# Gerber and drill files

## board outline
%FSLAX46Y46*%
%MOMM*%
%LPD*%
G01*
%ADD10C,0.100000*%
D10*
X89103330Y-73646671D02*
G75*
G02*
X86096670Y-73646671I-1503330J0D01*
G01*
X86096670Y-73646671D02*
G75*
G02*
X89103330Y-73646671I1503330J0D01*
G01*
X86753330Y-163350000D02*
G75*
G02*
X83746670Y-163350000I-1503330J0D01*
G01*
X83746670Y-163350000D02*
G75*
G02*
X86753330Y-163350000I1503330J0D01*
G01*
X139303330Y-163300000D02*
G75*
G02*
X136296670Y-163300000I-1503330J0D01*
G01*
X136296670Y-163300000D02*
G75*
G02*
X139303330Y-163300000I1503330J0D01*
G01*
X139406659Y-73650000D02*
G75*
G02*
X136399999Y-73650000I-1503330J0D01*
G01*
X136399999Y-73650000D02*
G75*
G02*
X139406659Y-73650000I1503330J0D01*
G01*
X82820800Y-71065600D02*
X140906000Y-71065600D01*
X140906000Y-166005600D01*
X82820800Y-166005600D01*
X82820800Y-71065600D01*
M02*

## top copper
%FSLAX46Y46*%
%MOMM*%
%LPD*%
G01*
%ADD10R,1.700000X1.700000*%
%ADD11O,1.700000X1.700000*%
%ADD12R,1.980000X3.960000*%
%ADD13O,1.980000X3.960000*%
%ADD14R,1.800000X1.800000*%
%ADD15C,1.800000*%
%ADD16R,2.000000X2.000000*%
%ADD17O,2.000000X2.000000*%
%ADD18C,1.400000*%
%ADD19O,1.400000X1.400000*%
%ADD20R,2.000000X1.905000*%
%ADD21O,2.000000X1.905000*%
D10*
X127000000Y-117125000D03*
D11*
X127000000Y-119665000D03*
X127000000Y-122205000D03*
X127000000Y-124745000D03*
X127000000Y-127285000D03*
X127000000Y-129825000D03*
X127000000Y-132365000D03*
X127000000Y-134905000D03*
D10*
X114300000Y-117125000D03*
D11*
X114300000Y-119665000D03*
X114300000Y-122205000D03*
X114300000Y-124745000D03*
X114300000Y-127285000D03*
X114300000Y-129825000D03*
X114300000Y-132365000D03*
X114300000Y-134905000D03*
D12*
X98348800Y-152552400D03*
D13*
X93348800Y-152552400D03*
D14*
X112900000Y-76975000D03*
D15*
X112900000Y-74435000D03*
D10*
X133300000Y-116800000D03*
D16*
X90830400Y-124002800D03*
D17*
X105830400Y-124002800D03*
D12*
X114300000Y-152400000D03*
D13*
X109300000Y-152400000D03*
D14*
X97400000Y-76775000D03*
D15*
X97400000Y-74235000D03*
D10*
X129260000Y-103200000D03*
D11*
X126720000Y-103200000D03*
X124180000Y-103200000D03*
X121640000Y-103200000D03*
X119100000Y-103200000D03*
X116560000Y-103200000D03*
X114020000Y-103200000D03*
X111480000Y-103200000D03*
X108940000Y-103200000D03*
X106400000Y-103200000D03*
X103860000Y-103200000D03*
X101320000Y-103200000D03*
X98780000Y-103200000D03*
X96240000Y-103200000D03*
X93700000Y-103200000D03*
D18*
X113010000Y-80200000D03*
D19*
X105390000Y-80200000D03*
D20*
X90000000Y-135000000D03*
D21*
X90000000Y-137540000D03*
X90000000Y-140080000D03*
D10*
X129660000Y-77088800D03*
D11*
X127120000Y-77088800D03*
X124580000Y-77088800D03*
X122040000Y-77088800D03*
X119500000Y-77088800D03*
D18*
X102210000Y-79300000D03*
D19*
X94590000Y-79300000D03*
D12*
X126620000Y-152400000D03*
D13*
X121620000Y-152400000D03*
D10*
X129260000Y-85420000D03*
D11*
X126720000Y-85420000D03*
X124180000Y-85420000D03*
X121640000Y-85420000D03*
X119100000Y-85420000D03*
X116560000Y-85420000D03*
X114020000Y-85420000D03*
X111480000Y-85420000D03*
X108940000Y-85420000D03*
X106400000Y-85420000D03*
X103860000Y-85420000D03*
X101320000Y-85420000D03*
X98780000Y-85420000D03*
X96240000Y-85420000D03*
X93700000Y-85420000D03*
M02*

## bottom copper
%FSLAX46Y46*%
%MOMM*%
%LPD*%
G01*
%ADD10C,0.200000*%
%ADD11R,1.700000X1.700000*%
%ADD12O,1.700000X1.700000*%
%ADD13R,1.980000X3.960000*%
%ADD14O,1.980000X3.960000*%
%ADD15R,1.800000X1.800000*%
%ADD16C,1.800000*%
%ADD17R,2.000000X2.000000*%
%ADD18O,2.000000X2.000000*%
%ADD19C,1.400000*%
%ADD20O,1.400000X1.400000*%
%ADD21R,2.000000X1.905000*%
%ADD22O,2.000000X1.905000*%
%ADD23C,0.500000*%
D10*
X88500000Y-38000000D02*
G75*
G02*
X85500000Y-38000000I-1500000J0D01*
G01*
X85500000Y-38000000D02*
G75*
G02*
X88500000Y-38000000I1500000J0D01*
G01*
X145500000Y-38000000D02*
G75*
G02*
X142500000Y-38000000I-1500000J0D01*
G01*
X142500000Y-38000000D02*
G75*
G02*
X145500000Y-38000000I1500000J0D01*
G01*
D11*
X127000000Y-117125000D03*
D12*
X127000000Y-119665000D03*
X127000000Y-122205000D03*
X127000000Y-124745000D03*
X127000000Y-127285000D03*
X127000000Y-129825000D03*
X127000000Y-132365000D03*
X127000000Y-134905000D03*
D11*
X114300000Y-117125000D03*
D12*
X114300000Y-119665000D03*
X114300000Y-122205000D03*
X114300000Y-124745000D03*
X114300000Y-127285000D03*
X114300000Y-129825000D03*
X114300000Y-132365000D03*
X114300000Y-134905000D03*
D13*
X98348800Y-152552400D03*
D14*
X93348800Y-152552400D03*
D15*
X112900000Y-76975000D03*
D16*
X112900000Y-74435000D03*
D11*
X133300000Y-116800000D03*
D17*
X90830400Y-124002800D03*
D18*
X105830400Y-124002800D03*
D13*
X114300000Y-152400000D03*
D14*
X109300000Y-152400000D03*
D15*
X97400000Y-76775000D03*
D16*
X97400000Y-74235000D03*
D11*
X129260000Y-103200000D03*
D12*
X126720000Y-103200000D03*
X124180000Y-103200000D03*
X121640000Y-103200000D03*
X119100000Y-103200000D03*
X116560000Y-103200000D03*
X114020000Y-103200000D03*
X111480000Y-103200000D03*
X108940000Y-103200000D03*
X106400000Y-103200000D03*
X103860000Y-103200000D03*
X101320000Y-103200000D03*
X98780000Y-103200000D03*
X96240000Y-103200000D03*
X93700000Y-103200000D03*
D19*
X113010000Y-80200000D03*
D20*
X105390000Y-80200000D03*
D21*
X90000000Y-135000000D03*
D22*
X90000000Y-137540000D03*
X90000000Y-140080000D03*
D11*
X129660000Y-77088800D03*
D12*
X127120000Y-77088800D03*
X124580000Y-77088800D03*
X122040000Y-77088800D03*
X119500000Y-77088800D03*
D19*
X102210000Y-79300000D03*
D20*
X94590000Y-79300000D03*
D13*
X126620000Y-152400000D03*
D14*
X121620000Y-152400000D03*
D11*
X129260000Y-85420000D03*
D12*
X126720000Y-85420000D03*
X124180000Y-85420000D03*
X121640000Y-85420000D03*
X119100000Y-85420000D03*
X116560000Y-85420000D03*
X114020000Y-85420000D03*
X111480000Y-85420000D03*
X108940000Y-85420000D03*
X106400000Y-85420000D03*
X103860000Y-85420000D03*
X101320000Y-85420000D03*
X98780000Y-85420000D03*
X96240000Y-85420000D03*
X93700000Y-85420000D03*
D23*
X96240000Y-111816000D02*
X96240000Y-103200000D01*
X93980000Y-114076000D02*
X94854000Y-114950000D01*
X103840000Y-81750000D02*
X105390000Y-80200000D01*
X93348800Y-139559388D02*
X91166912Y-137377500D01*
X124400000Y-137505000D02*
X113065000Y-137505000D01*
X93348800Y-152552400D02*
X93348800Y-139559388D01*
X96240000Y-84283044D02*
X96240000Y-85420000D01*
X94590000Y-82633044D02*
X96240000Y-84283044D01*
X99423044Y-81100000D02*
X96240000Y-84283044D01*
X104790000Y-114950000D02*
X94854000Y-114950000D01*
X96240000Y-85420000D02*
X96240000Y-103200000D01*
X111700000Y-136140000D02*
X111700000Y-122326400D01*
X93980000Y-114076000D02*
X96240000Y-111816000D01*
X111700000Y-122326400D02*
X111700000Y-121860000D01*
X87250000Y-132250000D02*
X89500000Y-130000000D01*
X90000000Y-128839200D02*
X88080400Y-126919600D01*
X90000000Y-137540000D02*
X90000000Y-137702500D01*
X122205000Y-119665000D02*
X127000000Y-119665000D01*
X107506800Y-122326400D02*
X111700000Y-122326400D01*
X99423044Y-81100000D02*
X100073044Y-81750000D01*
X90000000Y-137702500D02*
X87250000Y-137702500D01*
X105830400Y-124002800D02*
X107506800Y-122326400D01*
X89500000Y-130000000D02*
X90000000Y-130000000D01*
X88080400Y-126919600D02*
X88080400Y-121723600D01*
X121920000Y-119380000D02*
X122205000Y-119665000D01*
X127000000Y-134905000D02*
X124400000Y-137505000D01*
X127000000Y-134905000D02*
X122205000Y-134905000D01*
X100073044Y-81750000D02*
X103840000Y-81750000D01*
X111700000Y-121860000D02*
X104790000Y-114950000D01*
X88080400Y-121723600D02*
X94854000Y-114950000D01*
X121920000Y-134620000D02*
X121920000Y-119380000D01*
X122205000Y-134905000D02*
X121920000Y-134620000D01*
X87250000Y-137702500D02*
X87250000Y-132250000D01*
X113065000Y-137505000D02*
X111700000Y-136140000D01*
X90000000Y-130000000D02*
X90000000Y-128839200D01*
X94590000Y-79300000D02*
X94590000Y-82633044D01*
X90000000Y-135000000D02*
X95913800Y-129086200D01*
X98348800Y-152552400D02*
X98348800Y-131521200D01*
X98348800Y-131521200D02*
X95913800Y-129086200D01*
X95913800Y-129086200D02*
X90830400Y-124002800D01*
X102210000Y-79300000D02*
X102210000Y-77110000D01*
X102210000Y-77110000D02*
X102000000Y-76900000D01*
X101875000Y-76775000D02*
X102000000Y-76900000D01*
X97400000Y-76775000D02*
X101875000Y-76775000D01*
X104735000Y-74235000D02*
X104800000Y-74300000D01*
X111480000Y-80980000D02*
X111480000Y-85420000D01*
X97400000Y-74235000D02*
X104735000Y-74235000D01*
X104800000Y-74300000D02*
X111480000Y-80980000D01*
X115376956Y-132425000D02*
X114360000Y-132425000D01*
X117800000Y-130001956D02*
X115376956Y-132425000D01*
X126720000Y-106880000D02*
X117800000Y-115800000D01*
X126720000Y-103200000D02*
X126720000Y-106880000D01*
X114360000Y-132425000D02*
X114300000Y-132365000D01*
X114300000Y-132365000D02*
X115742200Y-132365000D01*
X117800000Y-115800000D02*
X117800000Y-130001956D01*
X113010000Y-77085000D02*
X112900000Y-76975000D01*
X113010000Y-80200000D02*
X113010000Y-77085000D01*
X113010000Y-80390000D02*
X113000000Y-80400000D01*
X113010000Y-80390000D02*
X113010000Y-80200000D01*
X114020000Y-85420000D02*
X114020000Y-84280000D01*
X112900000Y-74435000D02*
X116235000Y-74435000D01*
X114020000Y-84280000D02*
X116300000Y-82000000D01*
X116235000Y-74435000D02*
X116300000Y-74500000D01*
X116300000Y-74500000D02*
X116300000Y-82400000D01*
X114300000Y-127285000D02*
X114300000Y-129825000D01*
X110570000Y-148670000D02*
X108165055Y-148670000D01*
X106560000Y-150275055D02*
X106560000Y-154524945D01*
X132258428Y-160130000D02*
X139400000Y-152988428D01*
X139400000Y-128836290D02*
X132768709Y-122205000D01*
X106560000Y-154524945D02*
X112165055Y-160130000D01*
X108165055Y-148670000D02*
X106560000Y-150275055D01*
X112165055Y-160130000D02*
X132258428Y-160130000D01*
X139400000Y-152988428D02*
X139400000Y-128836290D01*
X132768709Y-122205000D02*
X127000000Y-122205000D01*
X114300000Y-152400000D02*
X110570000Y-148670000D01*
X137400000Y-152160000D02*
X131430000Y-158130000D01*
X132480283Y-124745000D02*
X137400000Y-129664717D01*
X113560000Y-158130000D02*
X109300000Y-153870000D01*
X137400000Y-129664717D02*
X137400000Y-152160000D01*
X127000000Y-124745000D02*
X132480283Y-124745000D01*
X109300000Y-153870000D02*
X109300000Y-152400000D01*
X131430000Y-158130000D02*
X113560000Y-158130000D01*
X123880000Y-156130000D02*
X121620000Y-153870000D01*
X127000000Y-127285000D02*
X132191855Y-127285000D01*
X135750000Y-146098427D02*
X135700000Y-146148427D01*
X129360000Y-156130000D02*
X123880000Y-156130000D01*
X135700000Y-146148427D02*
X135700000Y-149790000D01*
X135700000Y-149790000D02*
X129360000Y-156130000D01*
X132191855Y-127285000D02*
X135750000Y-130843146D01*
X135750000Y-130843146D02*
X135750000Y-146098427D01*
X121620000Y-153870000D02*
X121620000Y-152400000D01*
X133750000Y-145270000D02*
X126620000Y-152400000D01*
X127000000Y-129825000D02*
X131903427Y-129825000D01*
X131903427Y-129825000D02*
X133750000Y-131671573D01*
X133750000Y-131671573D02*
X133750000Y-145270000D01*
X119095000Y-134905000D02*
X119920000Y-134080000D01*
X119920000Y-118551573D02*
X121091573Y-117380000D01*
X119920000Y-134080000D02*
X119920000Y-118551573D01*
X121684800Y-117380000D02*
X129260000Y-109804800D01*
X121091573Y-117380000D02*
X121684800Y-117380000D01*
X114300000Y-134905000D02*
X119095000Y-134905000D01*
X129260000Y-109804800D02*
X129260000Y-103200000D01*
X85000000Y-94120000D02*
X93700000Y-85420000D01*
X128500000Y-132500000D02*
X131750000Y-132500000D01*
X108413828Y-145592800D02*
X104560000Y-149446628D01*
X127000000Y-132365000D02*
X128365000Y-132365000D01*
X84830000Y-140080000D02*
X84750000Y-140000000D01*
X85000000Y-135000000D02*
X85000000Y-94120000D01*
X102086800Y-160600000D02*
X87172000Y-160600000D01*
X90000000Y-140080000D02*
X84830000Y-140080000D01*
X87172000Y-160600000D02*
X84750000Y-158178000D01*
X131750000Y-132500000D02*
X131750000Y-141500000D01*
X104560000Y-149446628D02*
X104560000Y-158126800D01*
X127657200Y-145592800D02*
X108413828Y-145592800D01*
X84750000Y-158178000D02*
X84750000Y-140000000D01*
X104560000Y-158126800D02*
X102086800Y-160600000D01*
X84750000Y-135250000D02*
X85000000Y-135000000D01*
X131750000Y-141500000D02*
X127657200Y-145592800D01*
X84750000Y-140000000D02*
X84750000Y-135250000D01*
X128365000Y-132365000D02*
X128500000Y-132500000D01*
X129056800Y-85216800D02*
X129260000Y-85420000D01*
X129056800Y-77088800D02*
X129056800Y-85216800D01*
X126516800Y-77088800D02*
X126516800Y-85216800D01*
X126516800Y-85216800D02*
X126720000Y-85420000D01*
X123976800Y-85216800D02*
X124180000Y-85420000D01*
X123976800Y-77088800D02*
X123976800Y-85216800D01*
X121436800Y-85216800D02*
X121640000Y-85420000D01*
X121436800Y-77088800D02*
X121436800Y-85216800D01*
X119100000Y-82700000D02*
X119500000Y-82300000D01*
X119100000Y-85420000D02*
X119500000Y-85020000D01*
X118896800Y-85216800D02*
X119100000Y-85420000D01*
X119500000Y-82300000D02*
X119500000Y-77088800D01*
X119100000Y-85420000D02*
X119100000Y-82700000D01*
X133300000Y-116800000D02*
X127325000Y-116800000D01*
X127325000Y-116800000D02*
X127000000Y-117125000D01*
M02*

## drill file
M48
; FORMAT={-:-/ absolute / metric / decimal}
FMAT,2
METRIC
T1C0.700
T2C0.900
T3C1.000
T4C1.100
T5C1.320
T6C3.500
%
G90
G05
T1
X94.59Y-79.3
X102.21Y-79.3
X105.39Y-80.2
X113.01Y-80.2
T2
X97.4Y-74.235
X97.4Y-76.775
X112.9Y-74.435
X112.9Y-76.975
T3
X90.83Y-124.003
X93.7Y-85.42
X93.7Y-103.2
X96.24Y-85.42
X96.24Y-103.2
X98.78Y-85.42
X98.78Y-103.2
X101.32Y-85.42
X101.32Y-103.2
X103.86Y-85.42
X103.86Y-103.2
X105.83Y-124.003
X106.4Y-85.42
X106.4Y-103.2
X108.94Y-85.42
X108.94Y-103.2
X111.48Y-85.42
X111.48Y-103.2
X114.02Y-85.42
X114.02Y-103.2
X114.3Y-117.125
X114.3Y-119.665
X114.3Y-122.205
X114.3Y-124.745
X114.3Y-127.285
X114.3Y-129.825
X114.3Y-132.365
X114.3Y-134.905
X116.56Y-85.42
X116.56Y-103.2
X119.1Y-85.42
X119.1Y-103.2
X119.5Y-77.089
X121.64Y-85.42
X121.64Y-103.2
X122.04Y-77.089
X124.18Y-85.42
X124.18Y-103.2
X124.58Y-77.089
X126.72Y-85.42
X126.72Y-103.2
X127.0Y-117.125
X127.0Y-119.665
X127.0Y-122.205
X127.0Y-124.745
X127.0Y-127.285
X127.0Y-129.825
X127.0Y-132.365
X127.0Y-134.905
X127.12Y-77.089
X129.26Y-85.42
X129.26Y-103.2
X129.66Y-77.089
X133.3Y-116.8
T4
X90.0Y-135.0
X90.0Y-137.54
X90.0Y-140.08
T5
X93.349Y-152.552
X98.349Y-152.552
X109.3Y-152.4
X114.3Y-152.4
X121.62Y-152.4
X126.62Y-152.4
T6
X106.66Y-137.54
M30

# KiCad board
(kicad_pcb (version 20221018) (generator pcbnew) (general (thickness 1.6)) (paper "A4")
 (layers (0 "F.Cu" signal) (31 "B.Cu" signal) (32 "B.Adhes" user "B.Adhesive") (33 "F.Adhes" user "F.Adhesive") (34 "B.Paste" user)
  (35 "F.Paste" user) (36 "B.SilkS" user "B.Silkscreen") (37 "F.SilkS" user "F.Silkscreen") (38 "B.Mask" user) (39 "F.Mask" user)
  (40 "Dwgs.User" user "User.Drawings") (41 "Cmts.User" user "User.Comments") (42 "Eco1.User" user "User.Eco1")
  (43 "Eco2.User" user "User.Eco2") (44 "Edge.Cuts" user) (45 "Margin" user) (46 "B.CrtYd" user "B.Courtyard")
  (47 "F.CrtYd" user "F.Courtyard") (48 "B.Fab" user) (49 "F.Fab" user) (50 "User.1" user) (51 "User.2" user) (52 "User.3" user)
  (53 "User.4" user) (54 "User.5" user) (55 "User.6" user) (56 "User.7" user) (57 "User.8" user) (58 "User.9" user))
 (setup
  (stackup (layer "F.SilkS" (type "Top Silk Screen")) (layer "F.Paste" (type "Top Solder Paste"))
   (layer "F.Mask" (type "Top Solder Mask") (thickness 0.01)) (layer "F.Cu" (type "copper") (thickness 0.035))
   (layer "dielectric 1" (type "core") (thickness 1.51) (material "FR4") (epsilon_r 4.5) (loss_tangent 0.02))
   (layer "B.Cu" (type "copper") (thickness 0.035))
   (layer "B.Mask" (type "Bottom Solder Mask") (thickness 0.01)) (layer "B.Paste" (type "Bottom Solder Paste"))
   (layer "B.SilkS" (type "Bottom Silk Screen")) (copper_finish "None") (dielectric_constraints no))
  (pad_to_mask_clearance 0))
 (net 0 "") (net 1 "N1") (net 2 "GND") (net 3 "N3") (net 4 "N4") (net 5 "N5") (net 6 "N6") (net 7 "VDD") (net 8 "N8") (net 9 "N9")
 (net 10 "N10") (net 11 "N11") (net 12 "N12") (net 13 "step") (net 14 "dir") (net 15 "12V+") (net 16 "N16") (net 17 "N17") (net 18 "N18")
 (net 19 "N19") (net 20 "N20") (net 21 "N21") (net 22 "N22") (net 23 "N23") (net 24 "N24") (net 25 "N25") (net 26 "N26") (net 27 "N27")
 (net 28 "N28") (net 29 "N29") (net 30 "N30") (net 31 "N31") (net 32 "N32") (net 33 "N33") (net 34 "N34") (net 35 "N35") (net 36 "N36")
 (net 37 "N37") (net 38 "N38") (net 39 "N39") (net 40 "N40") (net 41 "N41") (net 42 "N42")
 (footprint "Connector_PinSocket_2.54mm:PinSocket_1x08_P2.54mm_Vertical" (layer "F.Cu") (at 127 117.125)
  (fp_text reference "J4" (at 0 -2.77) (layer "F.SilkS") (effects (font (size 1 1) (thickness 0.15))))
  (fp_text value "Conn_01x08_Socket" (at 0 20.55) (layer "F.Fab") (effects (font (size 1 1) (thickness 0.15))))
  (pad "1" thru_hole rect (at 0 0) (size 1.7 1.7) (drill 1) (layers "*.Cu" "*.Mask") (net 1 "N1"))
  (pad "2" thru_hole oval (at 0 2.54) (size 1.7 1.7) (drill 1) (layers "*.Cu" "*.Mask") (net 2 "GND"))
  (pad "3" thru_hole oval (at 0 5.08) (size 1.7 1.7) (drill 1) (layers "*.Cu" "*.Mask") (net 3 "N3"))
  (pad "4" thru_hole oval (at 0 7.62) (size 1.7 1.7) (drill 1) (layers "*.Cu" "*.Mask") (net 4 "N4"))
  (pad "5" thru_hole oval (at 0 10.16) (size 1.7 1.7) (drill 1) (layers "*.Cu" "*.Mask") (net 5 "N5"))
  (pad "6" thru_hole oval (at 0 12.7) (size 1.7 1.7) (drill 1) (layers "*.Cu" "*.Mask") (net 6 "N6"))
  (pad "7" thru_hole oval (at 0 15.24) (size 1.7 1.7) (drill 1) (layers "*.Cu" "*.Mask") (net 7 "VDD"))
  (pad "8" thru_hole oval (at 0 17.78) (size 1.7 1.7) (drill 1) (layers "*.Cu" "*.Mask") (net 2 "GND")))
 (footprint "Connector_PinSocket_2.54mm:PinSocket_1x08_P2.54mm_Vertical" (layer "F.Cu") (at 114.3 117.125)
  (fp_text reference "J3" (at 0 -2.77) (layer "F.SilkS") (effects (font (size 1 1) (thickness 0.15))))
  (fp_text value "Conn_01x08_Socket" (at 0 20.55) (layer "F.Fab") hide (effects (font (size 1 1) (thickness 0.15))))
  (pad "1" thru_hole rect (at 0 0) (size 1.7 1.7) (drill 1) (layers "*.Cu" "*.Mask") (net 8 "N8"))
  (pad "2" thru_hole oval (at 0 2.54) (size 1.7 1.7) (drill 1) (layers "*.Cu" "*.Mask") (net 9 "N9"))
  (pad "3" thru_hole oval (at 0 5.08) (size 1.7 1.7) (drill 1) (layers "*.Cu" "*.Mask") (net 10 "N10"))
  (pad "4" thru_hole oval (at 0 7.62) (size 1.7 1.7) (drill 1) (layers "*.Cu" "*.Mask") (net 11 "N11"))
  (pad "5" thru_hole oval (at 0 10.16) (size 1.7 1.7) (drill 1) (layers "*.Cu" "*.Mask") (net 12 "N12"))
  (pad "6" thru_hole oval (at 0 12.7) (size 1.7 1.7) (drill 1) (layers "*.Cu" "*.Mask") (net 12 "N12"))
  (pad "7" thru_hole oval (at 0 15.24) (size 1.7 1.7) (drill 1) (layers "*.Cu" "*.Mask") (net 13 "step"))
  (pad "8" thru_hole oval (at 0 17.78) (size 1.7 1.7) (drill 1) (layers "*.Cu" "*.Mask") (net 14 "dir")))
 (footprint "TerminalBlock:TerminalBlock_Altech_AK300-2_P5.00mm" (layer "F.Cu") (at 98.3488 152.5524 180)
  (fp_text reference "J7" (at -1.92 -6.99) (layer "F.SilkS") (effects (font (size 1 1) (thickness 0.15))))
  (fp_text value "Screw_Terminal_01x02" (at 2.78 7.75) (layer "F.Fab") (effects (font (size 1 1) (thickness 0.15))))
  (pad "1" thru_hole rect (at 0 0 180) (size 1.98 3.96) (drill 1.32) (layers "*.Cu" "*.Mask") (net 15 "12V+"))
  (pad "2" thru_hole oval (at 5 0 180) (size 1.98 3.96) (drill 1.32) (layers "*.Cu" "*.Mask") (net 2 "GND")))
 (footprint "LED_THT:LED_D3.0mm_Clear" (layer "F.Cu") (at 112.9 76.975 90)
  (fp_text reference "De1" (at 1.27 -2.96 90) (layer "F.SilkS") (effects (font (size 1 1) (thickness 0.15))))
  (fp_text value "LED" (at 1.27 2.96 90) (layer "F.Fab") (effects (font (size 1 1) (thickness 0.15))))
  (pad "1" thru_hole rect (at 0 0 90) (size 1.8 1.8) (drill 0.9) (layers "*.Cu" "*.Mask") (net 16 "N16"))
  (pad "2" thru_hole circle (at 2.54 0 90) (size 1.8 1.8) (drill 0.9) (layers "*.Cu" "*.Mask") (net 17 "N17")))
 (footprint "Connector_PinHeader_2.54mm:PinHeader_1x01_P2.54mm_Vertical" (layer "F.Cu") (at 133.3 116.8)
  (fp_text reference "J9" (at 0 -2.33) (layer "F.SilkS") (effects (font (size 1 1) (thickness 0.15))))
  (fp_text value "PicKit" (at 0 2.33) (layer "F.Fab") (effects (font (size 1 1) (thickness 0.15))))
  (pad "1" thru_hole rect (at 0 0) (size 1.7 1.7) (drill 1) (layers "*.Cu" "*.Mask") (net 1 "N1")))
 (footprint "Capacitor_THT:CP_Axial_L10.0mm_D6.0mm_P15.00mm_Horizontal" (layer "F.Cu") (at 90.8304 124.0028)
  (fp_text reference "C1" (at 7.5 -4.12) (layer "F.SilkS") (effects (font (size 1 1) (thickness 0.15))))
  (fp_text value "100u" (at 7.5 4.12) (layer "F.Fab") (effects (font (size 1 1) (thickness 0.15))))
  (pad "1" thru_hole rect (at 0 0) (size 2 2) (drill 1) (layers "*.Cu" "*.Mask") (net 15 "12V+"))
  (pad "2" thru_hole oval (at 15 0) (size 2 2) (drill 1) (layers "*.Cu" "*.Mask") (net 2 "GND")))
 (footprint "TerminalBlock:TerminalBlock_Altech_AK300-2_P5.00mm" (layer "F.Cu") (at 114.3 152.4 180)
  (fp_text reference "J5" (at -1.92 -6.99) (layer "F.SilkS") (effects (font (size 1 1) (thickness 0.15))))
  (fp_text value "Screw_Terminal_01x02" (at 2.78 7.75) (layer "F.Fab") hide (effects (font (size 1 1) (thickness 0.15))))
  (pad "1" thru_hole rect (at 0 0 180) (size 1.98 3.96) (drill 1.32) (layers "*.Cu" "*.Mask") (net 3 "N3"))
  (pad "2" thru_hole oval (at 5 0 180) (size 1.98 3.96) (drill 1.32) (layers "*.Cu" "*.Mask") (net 4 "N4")))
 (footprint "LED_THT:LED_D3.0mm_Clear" (layer "F.Cu") (at 97.4 76.775 90)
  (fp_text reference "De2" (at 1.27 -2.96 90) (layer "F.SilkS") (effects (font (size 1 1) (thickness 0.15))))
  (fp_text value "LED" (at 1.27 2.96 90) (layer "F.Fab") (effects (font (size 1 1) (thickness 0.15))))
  (pad "1" thru_hole rect (at 0 0 90) (size 1.8 1.8) (drill 0.9) (layers "*.Cu" "*.Mask") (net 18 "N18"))
  (pad "2" thru_hole circle (at 2.54 0 90) (size 1.8 1.8) (drill 0.9) (layers "*.Cu" "*.Mask") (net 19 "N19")))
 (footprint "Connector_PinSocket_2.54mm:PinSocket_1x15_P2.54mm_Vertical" (layer "F.Cu") (at 129.26 103.2 -90)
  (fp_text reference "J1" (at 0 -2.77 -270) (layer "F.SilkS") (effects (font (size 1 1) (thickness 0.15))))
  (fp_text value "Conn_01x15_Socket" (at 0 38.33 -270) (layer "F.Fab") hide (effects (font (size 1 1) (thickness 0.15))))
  (pad "1" thru_hole rect (at 0 0 270) (size 1.7 1.7) (drill 1) (layers "*.Cu" "*.Mask") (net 14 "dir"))
  (pad "2" thru_hole oval (at 0 2.54 270) (size 1.7 1.7) (drill 1) (layers "*.Cu" "*.Mask") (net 13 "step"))
  (pad "3" thru_hole oval (at 0 5.08 270) (size 1.7 1.7) (drill 1) (layers "*.Cu" "*.Mask") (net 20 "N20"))
  (pad "4" thru_hole oval (at 0 7.62 270) (size 1.7 1.7) (drill 1) (layers "*.Cu" "*.Mask") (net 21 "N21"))
  (pad "5" thru_hole oval (at 0 10.16 270) (size 1.7 1.7) (drill 1) (layers "*.Cu" "*.Mask") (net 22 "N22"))
  (pad "6" thru_hole oval (at 0 12.7 270) (size 1.7 1.7) (drill 1) (layers "*.Cu" "*.Mask") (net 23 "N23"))
  (pad "7" thru_hole oval (at 0 15.24 270) (size 1.7 1.7) (drill 1) (layers "*.Cu" "*.Mask") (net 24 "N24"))
  (pad "8" thru_hole oval (at 0 17.78 270) (size 1.7 1.7) (drill 1) (layers "*.Cu" "*.Mask") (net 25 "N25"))
  (pad "9" thru_hole oval (at 0 20.32 270) (size 1.7 1.7) (drill 1) (layers "*.Cu" "*.Mask") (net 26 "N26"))
  (pad "10" thru_hole oval (at 0 22.86 270) (size 1.7 1.7) (drill 1) (layers "*.Cu" "*.Mask") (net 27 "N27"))
  (pad "11" thru_hole oval (at 0 25.4 270) (size 1.7 1.7) (drill 1) (layers "*.Cu" "*.Mask") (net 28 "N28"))
  (pad "12" thru_hole oval (at 0 27.94 270) (size 1.7 1.7) (drill 1) (layers "*.Cu" "*.Mask") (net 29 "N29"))
  (pad "13" thru_hole oval (at 0 30.48 270) (size 1.7 1.7) (drill 1) (layers "*.Cu" "*.Mask") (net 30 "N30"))
  (pad "14" thru_hole oval (at 0 33.02 270) (size 1.7 1.7) (drill 1) (layers "*.Cu" "*.Mask") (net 2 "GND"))
  (pad "15" thru_hole oval (at 0 35.56 270) (size 1.7 1.7) (drill 1) (layers "*.Cu" "*.Mask") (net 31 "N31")))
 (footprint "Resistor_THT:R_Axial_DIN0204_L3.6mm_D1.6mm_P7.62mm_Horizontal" (layer "F.Cu") (at 113.01 80.2 180)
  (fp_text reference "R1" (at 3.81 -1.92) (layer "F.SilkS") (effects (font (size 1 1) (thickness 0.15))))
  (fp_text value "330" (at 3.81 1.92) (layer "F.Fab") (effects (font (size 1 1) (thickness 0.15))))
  (pad "1" thru_hole circle (at 0 0 180) (size 1.4 1.4) (drill 0.7) (layers "*.Cu" "*.Mask") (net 16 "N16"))
  (pad "2" thru_hole oval (at 7.62 0 180) (size 1.4 1.4) (drill 0.7) (layers "*.Cu" "*.Mask") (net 2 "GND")))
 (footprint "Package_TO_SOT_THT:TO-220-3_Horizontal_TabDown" (layer "F.Cu") (at 90 135 -90)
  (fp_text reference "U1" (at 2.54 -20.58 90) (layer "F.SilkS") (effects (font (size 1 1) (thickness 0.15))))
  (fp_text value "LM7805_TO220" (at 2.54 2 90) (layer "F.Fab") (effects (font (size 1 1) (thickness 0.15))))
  (pad "" np_thru_hole oval (at 2.54 -16.66 270) (size 3.5 3.5) (drill 3.5) (layers "*.Cu" "*.Mask"))
  (pad "1" thru_hole rect (at 0 0 270) (size 1.905 2) (drill 1.1) (layers "*.Cu" "*.Mask") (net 15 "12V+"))
  (pad "2" thru_hole oval (at 2.54 0 270) (size 1.905 2) (drill 1.1) (layers "*.Cu" "*.Mask") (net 2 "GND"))
  (pad "3" thru_hole oval (at 5.08 0 270) (size 1.905 2) (drill 1.1) (layers "*.Cu" "*.Mask") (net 7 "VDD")))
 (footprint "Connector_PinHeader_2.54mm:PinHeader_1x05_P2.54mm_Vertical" (layer "F.Cu") (at 129.66 77.0888 -90)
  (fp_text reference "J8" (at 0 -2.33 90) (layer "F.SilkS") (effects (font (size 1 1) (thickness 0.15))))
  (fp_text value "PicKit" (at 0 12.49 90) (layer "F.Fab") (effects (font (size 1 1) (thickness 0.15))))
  (pad "1" thru_hole rect (at 0 0 270) (size 1.7 1.7) (drill 1) (layers "*.Cu" "*.Mask") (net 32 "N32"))
  (pad "2" thru_hole oval (at 0 2.54 270) (size 1.7 1.7) (drill 1) (layers "*.Cu" "*.Mask") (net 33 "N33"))
  (pad "3" thru_hole oval (at 0 5.08 270) (size 1.7 1.7) (drill 1) (layers "*.Cu" "*.Mask") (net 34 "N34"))
  (pad "4" thru_hole oval (at 0 7.62 270) (size 1.7 1.7) (drill 1) (layers "*.Cu" "*.Mask") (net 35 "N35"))
  (pad "5" thru_hole oval (at 0 10.16 270) (size 1.7 1.7) (drill 1) (layers "*.Cu" "*.Mask") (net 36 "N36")))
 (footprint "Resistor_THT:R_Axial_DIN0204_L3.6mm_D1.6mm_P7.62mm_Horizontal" (layer "F.Cu") (at 102.21 79.3 180)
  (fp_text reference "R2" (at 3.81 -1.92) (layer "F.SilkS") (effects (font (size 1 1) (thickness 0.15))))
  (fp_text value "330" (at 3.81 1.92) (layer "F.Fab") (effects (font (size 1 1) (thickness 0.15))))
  (pad "1" thru_hole circle (at 0 0 180) (size 1.4 1.4) (drill 0.7) (layers "*.Cu" "*.Mask") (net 18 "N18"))
  (pad "2" thru_hole oval (at 7.62 0 180) (size 1.4 1.4) (drill 0.7) (layers "*.Cu" "*.Mask") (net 2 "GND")))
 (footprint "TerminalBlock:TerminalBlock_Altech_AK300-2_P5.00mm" (layer "F.Cu") (at 126.62 152.4 180)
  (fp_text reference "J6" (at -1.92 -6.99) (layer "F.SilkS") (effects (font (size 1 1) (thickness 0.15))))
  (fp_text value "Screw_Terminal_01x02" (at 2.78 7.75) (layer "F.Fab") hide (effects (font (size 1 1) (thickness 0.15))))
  (pad "1" thru_hole rect (at 0 0 180) (size 1.98 3.96) (drill 1.32) (layers "*.Cu" "*.Mask") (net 6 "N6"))
  (pad "2" thru_hole oval (at 5 0 180) (size 1.98 3.96) (drill 1.32) (layers "*.Cu" "*.Mask") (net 5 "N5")))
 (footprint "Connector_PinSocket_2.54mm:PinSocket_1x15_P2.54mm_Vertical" (layer "F.Cu") (at 129.26 85.42 -90)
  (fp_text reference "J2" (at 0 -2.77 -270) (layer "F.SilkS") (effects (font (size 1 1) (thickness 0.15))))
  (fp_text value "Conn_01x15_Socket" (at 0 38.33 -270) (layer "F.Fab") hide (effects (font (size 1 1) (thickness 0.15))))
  (pad "1" thru_hole rect (at 0 0 270) (size 1.7 1.7) (drill 1) (layers "*.Cu" "*.Mask") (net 32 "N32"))
  (pad "2" thru_hole oval (at 0 2.54 270) (size 1.7 1.7) (drill 1) (layers "*.Cu" "*.Mask") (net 33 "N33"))
  (pad "3" thru_hole oval (at 0 5.08 270) (size 1.7 1.7) (drill 1) (layers "*.Cu" "*.Mask") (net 34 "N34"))
  (pad "4" thru_hole oval (at 0 7.62 270) (size 1.7 1.7) (drill 1) (layers "*.Cu" "*.Mask") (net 35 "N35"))
  (pad "5" thru_hole oval (at 0 10.16 270) (size 1.7 1.7) (drill 1) (layers "*.Cu" "*.Mask") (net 36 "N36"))
  (pad "6" thru_hole oval (at 0 12.7 270) (size 1.7 1.7) (drill 1) (layers "*.Cu" "*.Mask") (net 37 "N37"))
  (pad "7" thru_hole oval (at 0 15.24 270) (size 1.7 1.7) (drill 1) (layers "*.Cu" "*.Mask") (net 17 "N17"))
  (pad "8" thru_hole oval (at 0 17.78 270) (size 1.7 1.7) (drill 1) (layers "*.Cu" "*.Mask") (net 19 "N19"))
  (pad "9" thru_hole oval (at 0 20.32 270) (size 1.7 1.7) (drill 1) (layers "*.Cu" "*.Mask") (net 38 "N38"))
  (pad "10" thru_hole oval (at 0 22.86 270) (size 1.7 1.7) (drill 1) (layers "*.Cu" "*.Mask") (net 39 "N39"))
  (pad "11" thru_hole oval (at 0 25.4 270) (size 1.7 1.7) (drill 1) (layers "*.Cu" "*.Mask") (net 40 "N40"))
  (pad "12" thru_hole oval (at 0 27.94 270) (size 1.7 1.7) (drill 1) (layers "*.Cu" "*.Mask") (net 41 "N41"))
  (pad "13" thru_hole oval (at 0 30.48 270) (size 1.7 1.7) (drill 1) (layers "*.Cu" "*.Mask") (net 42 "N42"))
  (pad "14" thru_hole oval (at 0 33.02 270) (size 1.7 1.7) (drill 1) (layers "*.Cu" "*.Mask") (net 2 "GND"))
  (pad "15" thru_hole oval (at 0 35.56 270) (size 1.7 1.7) (drill 1) (layers "*.Cu" "*.Mask") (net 7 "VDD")))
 (gr_circle (center 87 38) (end 88.5 38) (stroke (width 0.2) (type default)) (fill none) (layer "B.Cu"))
 (gr_circle (center 144 38) (end 145.5 38) (stroke (width 0.2) (type default)) (fill none) (layer "B.Cu"))
 (gr_circle (center 87.6 73.646671) (end 89.1 73.746671) (stroke (width 0.1) (type default)) (fill none) (layer "Edge.Cuts"))
 (gr_circle (center 85.25 163.35) (end 86.75 163.45) (stroke (width 0.1) (type default)) (fill none) (layer "Edge.Cuts"))
 (gr_circle (center 137.8 163.3) (end 139.3 163.4) (stroke (width 0.1) (type default)) (fill none) (layer "Edge.Cuts"))
 (gr_circle (center 137.903329 73.65) (end 139.403329 73.75) (stroke (width 0.1) (type default)) (fill none) (layer "Edge.Cuts"))
 (gr_rect (start 82.8208 71.0656) (end 140.906 166.0056) (stroke (width 0.1) (type default)) (fill none) (layer "Edge.Cuts"))
 (segment (start 96.24 111.816) (end 96.24 103.2) (width 0.5) (layer "B.Cu") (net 2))
 (segment (start 93.98 114.076) (end 94.854 114.95) (width 0.5) (layer "B.Cu") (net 2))
 (segment (start 103.84 81.75) (end 105.39 80.2) (width 0.5) (layer "B.Cu") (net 2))
 (segment (start 93.3488 139.559388) (end 91.166912 137.3775) (width 0.5) (layer "B.Cu") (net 2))
 (segment (start 124.4 137.505) (end 113.065 137.505) (width 0.5) (layer "B.Cu") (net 2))
 (segment (start 93.3488 152.5524) (end 93.3488 139.559388) (width 0.5) (layer "B.Cu") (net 2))
 (segment (start 96.24 84.283044) (end 96.24 85.42) (width 0.5) (layer "B.Cu") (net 2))
 (segment (start 94.59 82.633044) (end 96.24 84.283044) (width 0.5) (layer "B.Cu") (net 2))
 (segment (start 99.423044 81.1) (end 96.24 84.283044) (width 0.5) (layer "B.Cu") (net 2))
 (segment (start 104.79 114.95) (end 94.854 114.95) (width 0.5) (layer "B.Cu") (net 2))
 (segment (start 96.24 85.42) (end 96.24 103.2) (width 0.5) (layer "B.Cu") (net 2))
 (segment (start 111.7 136.14) (end 111.7 122.3264) (width 0.5) (layer "B.Cu") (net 2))
 (segment (start 93.98 114.076) (end 96.24 111.816) (width 0.5) (layer "B.Cu") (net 2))
 (segment (start 111.7 122.3264) (end 111.7 121.86) (width 0.5) (layer "B.Cu") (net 2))
 (segment (start 87.25 132.25) (end 89.5 130) (width 0.5) (layer "B.Cu") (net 2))
 (segment (start 90 128.8392) (end 88.0804 126.9196) (width 0.5) (layer "B.Cu") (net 2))
 (segment (start 90 137.54) (end 90 137.7025) (width 0.5) (layer "B.Cu") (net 2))
 (segment (start 122.205 119.665) (end 127 119.665) (width 0.5) (layer "B.Cu") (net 2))
 (segment (start 107.5068 122.3264) (end 111.7 122.3264) (width 0.5) (layer "B.Cu") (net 2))
 (segment (start 99.423044 81.1) (end 100.073044 81.75) (width 0.5) (layer "B.Cu") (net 2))
 (segment (start 90 137.7025) (end 87.25 137.7025) (width 0.5) (layer "B.Cu") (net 2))
 (segment (start 105.8304 124.0028) (end 107.5068 122.3264) (width 0.5) (layer "B.Cu") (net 2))
 (segment (start 89.5 130) (end 90 130) (width 0.5) (layer "B.Cu") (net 2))
 (segment (start 88.0804 126.9196) (end 88.0804 121.7236) (width 0.5) (layer "B.Cu") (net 2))
 (segment (start 121.92 119.38) (end 122.205 119.665) (width 0.5) (layer "B.Cu") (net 2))
 (segment (start 127 134.905) (end 124.4 137.505) (width 0.5) (layer "B.Cu") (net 2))
 (segment (start 127 134.905) (end 122.205 134.905) (width 0.5) (layer "B.Cu") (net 2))
 (segment (start 100.073044 81.75) (end 103.84 81.75) (width 0.5) (layer "B.Cu") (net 2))
 (segment (start 111.7 121.86) (end 104.79 114.95) (width 0.5) (layer "B.Cu") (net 2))
 (segment (start 88.0804 121.7236) (end 94.854 114.95) (width 0.5) (layer "B.Cu") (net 2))
 (segment (start 121.92 134.62) (end 121.92 119.38) (width 0.5) (layer "B.Cu") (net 2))
 (segment (start 122.205 134.905) (end 121.92 134.62) (width 0.5) (layer "B.Cu") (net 2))
 (segment (start 87.25 137.7025) (end 87.25 132.25) (width 0.5) (layer "B.Cu") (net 2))
 (segment (start 113.065 137.505) (end 111.7 136.14) (width 0.5) (layer "B.Cu") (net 2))
 (segment (start 90 130) (end 90 128.8392) (width 0.5) (layer "B.Cu") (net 2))
 (segment (start 94.59 79.3) (end 94.59 82.633044) (width 0.5) (layer "B.Cu") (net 2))
 (segment (start 90 135) (end 95.9138 129.0862) (width 0.5) (layer "B.Cu") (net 15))
 (segment (start 98.3488 152.5524) (end 98.3488 131.5212) (width 0.5) (layer "B.Cu") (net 15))
 (segment (start 98.3488 131.5212) (end 95.9138 129.0862) (width 0.5) (layer "B.Cu") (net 15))
 (segment (start 95.9138 129.0862) (end 90.8304 124.0028) (width 0.5) (layer "B.Cu") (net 15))
 (segment (start 102.21 79.3) (end 102.21 77.11) (width 0.5) (layer "B.Cu") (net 18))
 (segment (start 102.21 77.11) (end 102 76.9) (width 0.5) (layer "B.Cu") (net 18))
 (segment (start 101.875 76.775) (end 102 76.9) (width 0.5) (layer "B.Cu") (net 18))
 (segment (start 97.4 76.775) (end 101.875 76.775) (width 0.5) (layer "B.Cu") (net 18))
 (segment (start 104.735 74.235) (end 104.8 74.3) (width 0.5) (layer "B.Cu") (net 19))
 (segment (start 111.48 80.98) (end 111.48 85.42) (width 0.5) (layer "B.Cu") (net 19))
 (segment (start 97.4 74.235) (end 104.735 74.235) (width 0.5) (layer "B.Cu") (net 19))
 (segment (start 104.8 74.3) (end 111.48 80.98) (width 0.5) (layer "B.Cu") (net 19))
 (segment (start 115.376956 132.425) (end 114.36 132.425) (width 0.5) (layer "B.Cu") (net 13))
 (segment (start 117.8 130.001956) (end 115.376956 132.425) (width 0.5) (layer "B.Cu") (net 13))
 (segment (start 126.72 106.88) (end 117.8 115.8) (width 0.5) (layer "B.Cu") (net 13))
 (segment (start 126.72 103.2) (end 126.72 106.88) (width 0.5) (layer "B.Cu") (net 13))
 (segment (start 114.36 132.425) (end 114.3 132.365) (width 0.5) (layer "B.Cu") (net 13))
 (segment (start 114.3 132.365) (end 115.7422 132.365) (width 0.5) (layer "B.Cu") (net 13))
 (segment (start 117.8 115.8) (end 117.8 130.001956) (width 0.5) (layer "B.Cu") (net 13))
 (segment (start 113.01 77.085) (end 112.9 76.975) (width 0.5) (layer "B.Cu") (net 16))
 (segment (start 113.01 80.2) (end 113.01 77.085) (width 0.5) (layer "B.Cu") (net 16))
 (segment (start 113.01 80.39) (end 113 80.4) (width 0.5) (layer "B.Cu") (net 16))
 (segment (start 113.01 80.39) (end 113.01 80.2) (width 0.5) (layer "B.Cu") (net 16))
 (segment (start 114.02 85.42) (end 114.02 84.28) (width 0.5) (layer "B.Cu") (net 17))
 (segment (start 112.9 74.435) (end 116.235 74.435) (width 0.5) (layer "B.Cu") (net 17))
 (segment (start 114.02 84.28) (end 116.3 82) (width 0.5) (layer "B.Cu") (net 17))
 (segment (start 116.235 74.435) (end 116.3 74.5) (width 0.5) (layer "B.Cu") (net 17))
 (segment (start 116.3 74.5) (end 116.3 82.4) (width 0.5) (layer "B.Cu") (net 17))
 (segment (start 114.3 127.285) (end 114.3 129.825) (width 0.5) (layer "B.Cu") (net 12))
 (segment (start 110.57 148.67) (end 108.165055 148.67) (width 0.5) (layer "B.Cu") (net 3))
 (segment (start 106.56 150.275055) (end 106.56 154.524945) (width 0.5) (layer "B.Cu") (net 3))
 (segment (start 132.258428 160.13) (end 139.4 152.988428) (width 0.5) (layer "B.Cu") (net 3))
 (segment (start 139.4 128.83629) (end 132.768709 122.205) (width 0.5) (layer "B.Cu") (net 3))
 (segment (start 106.56 154.524945) (end 112.165055 160.13) (width 0.5) (layer "B.Cu") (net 3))
 (segment (start 108.165055 148.67) (end 106.56 150.275055) (width 0.5) (layer "B.Cu") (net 3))
 (segment (start 112.165055 160.13) (end 132.258428 160.13) (width 0.5) (layer "B.Cu") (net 3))
 (segment (start 139.4 152.988428) (end 139.4 128.83629) (width 0.5) (layer "B.Cu") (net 3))
 (segment (start 132.768709 122.205) (end 127 122.205) (width 0.5) (layer "B.Cu") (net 3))
 (segment (start 114.3 152.4) (end 110.57 148.67) (width 0.5) (layer "B.Cu") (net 3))
 (segment (start 137.4 152.16) (end 131.43 158.13) (width 0.5) (layer "B.Cu") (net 4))
 (segment (start 132.480283 124.745) (end 137.4 129.664717) (width 0.5) (layer "B.Cu") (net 4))
 (segment (start 113.56 158.13) (end 109.3 153.87) (width 0.5) (layer "B.Cu") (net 4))
 (segment (start 137.4 129.664717) (end 137.4 152.16) (width 0.5) (layer "B.Cu") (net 4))
 (segment (start 127 124.745) (end 132.480283 124.745) (width 0.5) (layer "B.Cu") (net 4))
 (segment (start 109.3 153.87) (end 109.3 152.4) (width 0.5) (layer "B.Cu") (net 4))
 (segment (start 131.43 158.13) (end 113.56 158.13) (width 0.5) (layer "B.Cu") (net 4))
 (segment (start 123.88 156.13) (end 121.62 153.87) (width 0.5) (layer "B.Cu") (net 5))
 (segment (start 127 127.285) (end 132.191855 127.285) (width 0.5) (layer "B.Cu") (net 5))
 (segment (start 135.75 146.098427) (end 135.7 146.148427) (width 0.5) (layer "B.Cu") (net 5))
 (segment (start 129.36 156.13) (end 123.88 156.13) (width 0.5) (layer "B.Cu") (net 5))
 (segment (start 135.7 146.148427) (end 135.7 149.79) (width 0.5) (layer "B.Cu") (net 5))
 (segment (start 135.7 149.79) (end 129.36 156.13) (width 0.5) (layer "B.Cu") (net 5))
 (segment (start 132.191855 127.285) (end 135.75 130.843146) (width 0.5) (layer "B.Cu") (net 5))
 (segment (start 135.75 130.843146) (end 135.75 146.098427) (width 0.5) (layer "B.Cu") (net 5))
 (segment (start 121.62 153.87) (end 121.62 152.4) (width 0.5) (layer "B.Cu") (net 5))
 (segment (start 133.75 145.27) (end 126.62 152.4) (width 0.5) (layer "B.Cu") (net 6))
 (segment (start 127 129.825) (end 131.903427 129.825) (width 0.5) (layer "B.Cu") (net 6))
 (segment (start 131.903427 129.825) (end 133.75 131.671573) (width 0.5) (layer "B.Cu") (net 6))
 (segment (start 133.75 131.671573) (end 133.75 145.27) (width 0.5) (layer "B.Cu") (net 6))
 (segment (start 119.095 134.905) (end 119.92 134.08) (width 0.5) (layer "B.Cu") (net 14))
 (segment (start 119.92 118.551573) (end 121.091573 117.38) (width 0.5) (layer "B.Cu") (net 14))
 (segment (start 119.92 134.08) (end 119.92 118.551573) (width 0.5) (layer "B.Cu") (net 14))
 (segment (start 121.6848 117.38) (end 129.26 109.8048) (width 0.5) (layer "B.Cu") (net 14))
 (segment (start 121.091573 117.38) (end 121.6848 117.38) (width 0.5) (layer "B.Cu") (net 14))
 (segment (start 114.3 134.905) (end 119.095 134.905) (width 0.5) (layer "B.Cu") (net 14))
 (segment (start 129.26 109.8048) (end 129.26 103.2) (width 0.5) (layer "B.Cu") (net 14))
 (segment (start 85 94.12) (end 93.7 85.42) (width 0.5) (layer "B.Cu") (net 7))
 (segment (start 128.5 132.5) (end 131.75 132.5) (width 0.5) (layer "B.Cu") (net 7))
 (segment (start 108.413828 145.5928) (end 104.56 149.446628) (width 0.5) (layer "B.Cu") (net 7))
 (segment (start 127 132.365) (end 128.365 132.365) (width 0.5) (layer "B.Cu") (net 7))
 (segment (start 84.83 140.08) (end 84.75 140) (width 0.5) (layer "B.Cu") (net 7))
 (segment (start 85 135) (end 85 94.12) (width 0.5) (layer "B.Cu") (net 7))
 (segment (start 102.0868 160.6) (end 87.172 160.6) (width 0.5) (layer "B.Cu") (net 7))
 (segment (start 90 140.08) (end 84.83 140.08) (width 0.5) (layer "B.Cu") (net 7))
 (segment (start 87.172 160.6) (end 84.75 158.178) (width 0.5) (layer "B.Cu") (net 7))
 (segment (start 131.75 132.5) (end 131.75 141.5) (width 0.5) (layer "B.Cu") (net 7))
 (segment (start 104.56 149.446628) (end 104.56 158.1268) (width 0.5) (layer "B.Cu") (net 7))
 (segment (start 127.6572 145.5928) (end 108.413828 145.5928) (width 0.5) (layer "B.Cu") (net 7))
 (segment (start 84.75 158.178) (end 84.75 140) (width 0.5) (layer "B.Cu") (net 7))
 (segment (start 104.56 158.1268) (end 102.0868 160.6) (width 0.5) (layer "B.Cu") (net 7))
 (segment (start 84.75 135.25) (end 85 135) (width 0.5) (layer "B.Cu") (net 7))
 (segment (start 131.75 141.5) (end 127.6572 145.5928) (width 0.5) (layer "B.Cu") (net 7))
 (segment (start 84.75 140) (end 84.75 135.25) (width 0.5) (layer "B.Cu") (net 7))
 (segment (start 128.365 132.365) (end 128.5 132.5) (width 0.5) (layer "B.Cu") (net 7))
 (segment (start 129.0568 85.2168) (end 129.26 85.42) (width 0.5) (layer "B.Cu") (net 32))
 (segment (start 129.0568 77.0888) (end 129.0568 85.2168) (width 0.5) (layer "B.Cu") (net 32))
 (segment (start 126.5168 77.0888) (end 126.5168 85.2168) (width 0.5) (layer "B.Cu") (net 33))
 (segment (start 126.5168 85.2168) (end 126.72 85.42) (width 0.5) (layer "B.Cu") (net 33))
 (segment (start 123.9768 85.2168) (end 124.18 85.42) (width 0.5) (layer "B.Cu") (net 34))
 (segment (start 123.9768 77.0888) (end 123.9768 85.2168) (width 0.5) (layer "B.Cu") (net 34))
 (segment (start 121.4368 85.2168) (end 121.64 85.42) (width 0.5) (layer "B.Cu") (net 35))
 (segment (start 121.4368 77.0888) (end 121.4368 85.2168) (width 0.5) (layer "B.Cu") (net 35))
 (segment (start 119.1 82.7) (end 119.5 82.3) (width 0.5) (layer "B.Cu") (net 36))
 (segment (start 119.1 85.42) (end 119.5 85.02) (width 0.5) (layer "B.Cu") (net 36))
 (segment (start 118.8968 85.2168) (end 119.1 85.42) (width 0.5) (layer "B.Cu") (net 36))
 (segment (start 119.5 82.3) (end 119.5 77.0888) (width 0.5) (layer "B.Cu") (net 36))
 (segment (start 119.1 85.42) (end 119.1 82.7) (width 0.5) (layer "B.Cu") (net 36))
 (segment (start 133.3 116.8) (end 127.325 116.8) (width 0.5) (layer "B.Cu") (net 1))
 (segment (start 127.325 116.8) (end 127 117.125) (width 0.5) (layer "B.Cu") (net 1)))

